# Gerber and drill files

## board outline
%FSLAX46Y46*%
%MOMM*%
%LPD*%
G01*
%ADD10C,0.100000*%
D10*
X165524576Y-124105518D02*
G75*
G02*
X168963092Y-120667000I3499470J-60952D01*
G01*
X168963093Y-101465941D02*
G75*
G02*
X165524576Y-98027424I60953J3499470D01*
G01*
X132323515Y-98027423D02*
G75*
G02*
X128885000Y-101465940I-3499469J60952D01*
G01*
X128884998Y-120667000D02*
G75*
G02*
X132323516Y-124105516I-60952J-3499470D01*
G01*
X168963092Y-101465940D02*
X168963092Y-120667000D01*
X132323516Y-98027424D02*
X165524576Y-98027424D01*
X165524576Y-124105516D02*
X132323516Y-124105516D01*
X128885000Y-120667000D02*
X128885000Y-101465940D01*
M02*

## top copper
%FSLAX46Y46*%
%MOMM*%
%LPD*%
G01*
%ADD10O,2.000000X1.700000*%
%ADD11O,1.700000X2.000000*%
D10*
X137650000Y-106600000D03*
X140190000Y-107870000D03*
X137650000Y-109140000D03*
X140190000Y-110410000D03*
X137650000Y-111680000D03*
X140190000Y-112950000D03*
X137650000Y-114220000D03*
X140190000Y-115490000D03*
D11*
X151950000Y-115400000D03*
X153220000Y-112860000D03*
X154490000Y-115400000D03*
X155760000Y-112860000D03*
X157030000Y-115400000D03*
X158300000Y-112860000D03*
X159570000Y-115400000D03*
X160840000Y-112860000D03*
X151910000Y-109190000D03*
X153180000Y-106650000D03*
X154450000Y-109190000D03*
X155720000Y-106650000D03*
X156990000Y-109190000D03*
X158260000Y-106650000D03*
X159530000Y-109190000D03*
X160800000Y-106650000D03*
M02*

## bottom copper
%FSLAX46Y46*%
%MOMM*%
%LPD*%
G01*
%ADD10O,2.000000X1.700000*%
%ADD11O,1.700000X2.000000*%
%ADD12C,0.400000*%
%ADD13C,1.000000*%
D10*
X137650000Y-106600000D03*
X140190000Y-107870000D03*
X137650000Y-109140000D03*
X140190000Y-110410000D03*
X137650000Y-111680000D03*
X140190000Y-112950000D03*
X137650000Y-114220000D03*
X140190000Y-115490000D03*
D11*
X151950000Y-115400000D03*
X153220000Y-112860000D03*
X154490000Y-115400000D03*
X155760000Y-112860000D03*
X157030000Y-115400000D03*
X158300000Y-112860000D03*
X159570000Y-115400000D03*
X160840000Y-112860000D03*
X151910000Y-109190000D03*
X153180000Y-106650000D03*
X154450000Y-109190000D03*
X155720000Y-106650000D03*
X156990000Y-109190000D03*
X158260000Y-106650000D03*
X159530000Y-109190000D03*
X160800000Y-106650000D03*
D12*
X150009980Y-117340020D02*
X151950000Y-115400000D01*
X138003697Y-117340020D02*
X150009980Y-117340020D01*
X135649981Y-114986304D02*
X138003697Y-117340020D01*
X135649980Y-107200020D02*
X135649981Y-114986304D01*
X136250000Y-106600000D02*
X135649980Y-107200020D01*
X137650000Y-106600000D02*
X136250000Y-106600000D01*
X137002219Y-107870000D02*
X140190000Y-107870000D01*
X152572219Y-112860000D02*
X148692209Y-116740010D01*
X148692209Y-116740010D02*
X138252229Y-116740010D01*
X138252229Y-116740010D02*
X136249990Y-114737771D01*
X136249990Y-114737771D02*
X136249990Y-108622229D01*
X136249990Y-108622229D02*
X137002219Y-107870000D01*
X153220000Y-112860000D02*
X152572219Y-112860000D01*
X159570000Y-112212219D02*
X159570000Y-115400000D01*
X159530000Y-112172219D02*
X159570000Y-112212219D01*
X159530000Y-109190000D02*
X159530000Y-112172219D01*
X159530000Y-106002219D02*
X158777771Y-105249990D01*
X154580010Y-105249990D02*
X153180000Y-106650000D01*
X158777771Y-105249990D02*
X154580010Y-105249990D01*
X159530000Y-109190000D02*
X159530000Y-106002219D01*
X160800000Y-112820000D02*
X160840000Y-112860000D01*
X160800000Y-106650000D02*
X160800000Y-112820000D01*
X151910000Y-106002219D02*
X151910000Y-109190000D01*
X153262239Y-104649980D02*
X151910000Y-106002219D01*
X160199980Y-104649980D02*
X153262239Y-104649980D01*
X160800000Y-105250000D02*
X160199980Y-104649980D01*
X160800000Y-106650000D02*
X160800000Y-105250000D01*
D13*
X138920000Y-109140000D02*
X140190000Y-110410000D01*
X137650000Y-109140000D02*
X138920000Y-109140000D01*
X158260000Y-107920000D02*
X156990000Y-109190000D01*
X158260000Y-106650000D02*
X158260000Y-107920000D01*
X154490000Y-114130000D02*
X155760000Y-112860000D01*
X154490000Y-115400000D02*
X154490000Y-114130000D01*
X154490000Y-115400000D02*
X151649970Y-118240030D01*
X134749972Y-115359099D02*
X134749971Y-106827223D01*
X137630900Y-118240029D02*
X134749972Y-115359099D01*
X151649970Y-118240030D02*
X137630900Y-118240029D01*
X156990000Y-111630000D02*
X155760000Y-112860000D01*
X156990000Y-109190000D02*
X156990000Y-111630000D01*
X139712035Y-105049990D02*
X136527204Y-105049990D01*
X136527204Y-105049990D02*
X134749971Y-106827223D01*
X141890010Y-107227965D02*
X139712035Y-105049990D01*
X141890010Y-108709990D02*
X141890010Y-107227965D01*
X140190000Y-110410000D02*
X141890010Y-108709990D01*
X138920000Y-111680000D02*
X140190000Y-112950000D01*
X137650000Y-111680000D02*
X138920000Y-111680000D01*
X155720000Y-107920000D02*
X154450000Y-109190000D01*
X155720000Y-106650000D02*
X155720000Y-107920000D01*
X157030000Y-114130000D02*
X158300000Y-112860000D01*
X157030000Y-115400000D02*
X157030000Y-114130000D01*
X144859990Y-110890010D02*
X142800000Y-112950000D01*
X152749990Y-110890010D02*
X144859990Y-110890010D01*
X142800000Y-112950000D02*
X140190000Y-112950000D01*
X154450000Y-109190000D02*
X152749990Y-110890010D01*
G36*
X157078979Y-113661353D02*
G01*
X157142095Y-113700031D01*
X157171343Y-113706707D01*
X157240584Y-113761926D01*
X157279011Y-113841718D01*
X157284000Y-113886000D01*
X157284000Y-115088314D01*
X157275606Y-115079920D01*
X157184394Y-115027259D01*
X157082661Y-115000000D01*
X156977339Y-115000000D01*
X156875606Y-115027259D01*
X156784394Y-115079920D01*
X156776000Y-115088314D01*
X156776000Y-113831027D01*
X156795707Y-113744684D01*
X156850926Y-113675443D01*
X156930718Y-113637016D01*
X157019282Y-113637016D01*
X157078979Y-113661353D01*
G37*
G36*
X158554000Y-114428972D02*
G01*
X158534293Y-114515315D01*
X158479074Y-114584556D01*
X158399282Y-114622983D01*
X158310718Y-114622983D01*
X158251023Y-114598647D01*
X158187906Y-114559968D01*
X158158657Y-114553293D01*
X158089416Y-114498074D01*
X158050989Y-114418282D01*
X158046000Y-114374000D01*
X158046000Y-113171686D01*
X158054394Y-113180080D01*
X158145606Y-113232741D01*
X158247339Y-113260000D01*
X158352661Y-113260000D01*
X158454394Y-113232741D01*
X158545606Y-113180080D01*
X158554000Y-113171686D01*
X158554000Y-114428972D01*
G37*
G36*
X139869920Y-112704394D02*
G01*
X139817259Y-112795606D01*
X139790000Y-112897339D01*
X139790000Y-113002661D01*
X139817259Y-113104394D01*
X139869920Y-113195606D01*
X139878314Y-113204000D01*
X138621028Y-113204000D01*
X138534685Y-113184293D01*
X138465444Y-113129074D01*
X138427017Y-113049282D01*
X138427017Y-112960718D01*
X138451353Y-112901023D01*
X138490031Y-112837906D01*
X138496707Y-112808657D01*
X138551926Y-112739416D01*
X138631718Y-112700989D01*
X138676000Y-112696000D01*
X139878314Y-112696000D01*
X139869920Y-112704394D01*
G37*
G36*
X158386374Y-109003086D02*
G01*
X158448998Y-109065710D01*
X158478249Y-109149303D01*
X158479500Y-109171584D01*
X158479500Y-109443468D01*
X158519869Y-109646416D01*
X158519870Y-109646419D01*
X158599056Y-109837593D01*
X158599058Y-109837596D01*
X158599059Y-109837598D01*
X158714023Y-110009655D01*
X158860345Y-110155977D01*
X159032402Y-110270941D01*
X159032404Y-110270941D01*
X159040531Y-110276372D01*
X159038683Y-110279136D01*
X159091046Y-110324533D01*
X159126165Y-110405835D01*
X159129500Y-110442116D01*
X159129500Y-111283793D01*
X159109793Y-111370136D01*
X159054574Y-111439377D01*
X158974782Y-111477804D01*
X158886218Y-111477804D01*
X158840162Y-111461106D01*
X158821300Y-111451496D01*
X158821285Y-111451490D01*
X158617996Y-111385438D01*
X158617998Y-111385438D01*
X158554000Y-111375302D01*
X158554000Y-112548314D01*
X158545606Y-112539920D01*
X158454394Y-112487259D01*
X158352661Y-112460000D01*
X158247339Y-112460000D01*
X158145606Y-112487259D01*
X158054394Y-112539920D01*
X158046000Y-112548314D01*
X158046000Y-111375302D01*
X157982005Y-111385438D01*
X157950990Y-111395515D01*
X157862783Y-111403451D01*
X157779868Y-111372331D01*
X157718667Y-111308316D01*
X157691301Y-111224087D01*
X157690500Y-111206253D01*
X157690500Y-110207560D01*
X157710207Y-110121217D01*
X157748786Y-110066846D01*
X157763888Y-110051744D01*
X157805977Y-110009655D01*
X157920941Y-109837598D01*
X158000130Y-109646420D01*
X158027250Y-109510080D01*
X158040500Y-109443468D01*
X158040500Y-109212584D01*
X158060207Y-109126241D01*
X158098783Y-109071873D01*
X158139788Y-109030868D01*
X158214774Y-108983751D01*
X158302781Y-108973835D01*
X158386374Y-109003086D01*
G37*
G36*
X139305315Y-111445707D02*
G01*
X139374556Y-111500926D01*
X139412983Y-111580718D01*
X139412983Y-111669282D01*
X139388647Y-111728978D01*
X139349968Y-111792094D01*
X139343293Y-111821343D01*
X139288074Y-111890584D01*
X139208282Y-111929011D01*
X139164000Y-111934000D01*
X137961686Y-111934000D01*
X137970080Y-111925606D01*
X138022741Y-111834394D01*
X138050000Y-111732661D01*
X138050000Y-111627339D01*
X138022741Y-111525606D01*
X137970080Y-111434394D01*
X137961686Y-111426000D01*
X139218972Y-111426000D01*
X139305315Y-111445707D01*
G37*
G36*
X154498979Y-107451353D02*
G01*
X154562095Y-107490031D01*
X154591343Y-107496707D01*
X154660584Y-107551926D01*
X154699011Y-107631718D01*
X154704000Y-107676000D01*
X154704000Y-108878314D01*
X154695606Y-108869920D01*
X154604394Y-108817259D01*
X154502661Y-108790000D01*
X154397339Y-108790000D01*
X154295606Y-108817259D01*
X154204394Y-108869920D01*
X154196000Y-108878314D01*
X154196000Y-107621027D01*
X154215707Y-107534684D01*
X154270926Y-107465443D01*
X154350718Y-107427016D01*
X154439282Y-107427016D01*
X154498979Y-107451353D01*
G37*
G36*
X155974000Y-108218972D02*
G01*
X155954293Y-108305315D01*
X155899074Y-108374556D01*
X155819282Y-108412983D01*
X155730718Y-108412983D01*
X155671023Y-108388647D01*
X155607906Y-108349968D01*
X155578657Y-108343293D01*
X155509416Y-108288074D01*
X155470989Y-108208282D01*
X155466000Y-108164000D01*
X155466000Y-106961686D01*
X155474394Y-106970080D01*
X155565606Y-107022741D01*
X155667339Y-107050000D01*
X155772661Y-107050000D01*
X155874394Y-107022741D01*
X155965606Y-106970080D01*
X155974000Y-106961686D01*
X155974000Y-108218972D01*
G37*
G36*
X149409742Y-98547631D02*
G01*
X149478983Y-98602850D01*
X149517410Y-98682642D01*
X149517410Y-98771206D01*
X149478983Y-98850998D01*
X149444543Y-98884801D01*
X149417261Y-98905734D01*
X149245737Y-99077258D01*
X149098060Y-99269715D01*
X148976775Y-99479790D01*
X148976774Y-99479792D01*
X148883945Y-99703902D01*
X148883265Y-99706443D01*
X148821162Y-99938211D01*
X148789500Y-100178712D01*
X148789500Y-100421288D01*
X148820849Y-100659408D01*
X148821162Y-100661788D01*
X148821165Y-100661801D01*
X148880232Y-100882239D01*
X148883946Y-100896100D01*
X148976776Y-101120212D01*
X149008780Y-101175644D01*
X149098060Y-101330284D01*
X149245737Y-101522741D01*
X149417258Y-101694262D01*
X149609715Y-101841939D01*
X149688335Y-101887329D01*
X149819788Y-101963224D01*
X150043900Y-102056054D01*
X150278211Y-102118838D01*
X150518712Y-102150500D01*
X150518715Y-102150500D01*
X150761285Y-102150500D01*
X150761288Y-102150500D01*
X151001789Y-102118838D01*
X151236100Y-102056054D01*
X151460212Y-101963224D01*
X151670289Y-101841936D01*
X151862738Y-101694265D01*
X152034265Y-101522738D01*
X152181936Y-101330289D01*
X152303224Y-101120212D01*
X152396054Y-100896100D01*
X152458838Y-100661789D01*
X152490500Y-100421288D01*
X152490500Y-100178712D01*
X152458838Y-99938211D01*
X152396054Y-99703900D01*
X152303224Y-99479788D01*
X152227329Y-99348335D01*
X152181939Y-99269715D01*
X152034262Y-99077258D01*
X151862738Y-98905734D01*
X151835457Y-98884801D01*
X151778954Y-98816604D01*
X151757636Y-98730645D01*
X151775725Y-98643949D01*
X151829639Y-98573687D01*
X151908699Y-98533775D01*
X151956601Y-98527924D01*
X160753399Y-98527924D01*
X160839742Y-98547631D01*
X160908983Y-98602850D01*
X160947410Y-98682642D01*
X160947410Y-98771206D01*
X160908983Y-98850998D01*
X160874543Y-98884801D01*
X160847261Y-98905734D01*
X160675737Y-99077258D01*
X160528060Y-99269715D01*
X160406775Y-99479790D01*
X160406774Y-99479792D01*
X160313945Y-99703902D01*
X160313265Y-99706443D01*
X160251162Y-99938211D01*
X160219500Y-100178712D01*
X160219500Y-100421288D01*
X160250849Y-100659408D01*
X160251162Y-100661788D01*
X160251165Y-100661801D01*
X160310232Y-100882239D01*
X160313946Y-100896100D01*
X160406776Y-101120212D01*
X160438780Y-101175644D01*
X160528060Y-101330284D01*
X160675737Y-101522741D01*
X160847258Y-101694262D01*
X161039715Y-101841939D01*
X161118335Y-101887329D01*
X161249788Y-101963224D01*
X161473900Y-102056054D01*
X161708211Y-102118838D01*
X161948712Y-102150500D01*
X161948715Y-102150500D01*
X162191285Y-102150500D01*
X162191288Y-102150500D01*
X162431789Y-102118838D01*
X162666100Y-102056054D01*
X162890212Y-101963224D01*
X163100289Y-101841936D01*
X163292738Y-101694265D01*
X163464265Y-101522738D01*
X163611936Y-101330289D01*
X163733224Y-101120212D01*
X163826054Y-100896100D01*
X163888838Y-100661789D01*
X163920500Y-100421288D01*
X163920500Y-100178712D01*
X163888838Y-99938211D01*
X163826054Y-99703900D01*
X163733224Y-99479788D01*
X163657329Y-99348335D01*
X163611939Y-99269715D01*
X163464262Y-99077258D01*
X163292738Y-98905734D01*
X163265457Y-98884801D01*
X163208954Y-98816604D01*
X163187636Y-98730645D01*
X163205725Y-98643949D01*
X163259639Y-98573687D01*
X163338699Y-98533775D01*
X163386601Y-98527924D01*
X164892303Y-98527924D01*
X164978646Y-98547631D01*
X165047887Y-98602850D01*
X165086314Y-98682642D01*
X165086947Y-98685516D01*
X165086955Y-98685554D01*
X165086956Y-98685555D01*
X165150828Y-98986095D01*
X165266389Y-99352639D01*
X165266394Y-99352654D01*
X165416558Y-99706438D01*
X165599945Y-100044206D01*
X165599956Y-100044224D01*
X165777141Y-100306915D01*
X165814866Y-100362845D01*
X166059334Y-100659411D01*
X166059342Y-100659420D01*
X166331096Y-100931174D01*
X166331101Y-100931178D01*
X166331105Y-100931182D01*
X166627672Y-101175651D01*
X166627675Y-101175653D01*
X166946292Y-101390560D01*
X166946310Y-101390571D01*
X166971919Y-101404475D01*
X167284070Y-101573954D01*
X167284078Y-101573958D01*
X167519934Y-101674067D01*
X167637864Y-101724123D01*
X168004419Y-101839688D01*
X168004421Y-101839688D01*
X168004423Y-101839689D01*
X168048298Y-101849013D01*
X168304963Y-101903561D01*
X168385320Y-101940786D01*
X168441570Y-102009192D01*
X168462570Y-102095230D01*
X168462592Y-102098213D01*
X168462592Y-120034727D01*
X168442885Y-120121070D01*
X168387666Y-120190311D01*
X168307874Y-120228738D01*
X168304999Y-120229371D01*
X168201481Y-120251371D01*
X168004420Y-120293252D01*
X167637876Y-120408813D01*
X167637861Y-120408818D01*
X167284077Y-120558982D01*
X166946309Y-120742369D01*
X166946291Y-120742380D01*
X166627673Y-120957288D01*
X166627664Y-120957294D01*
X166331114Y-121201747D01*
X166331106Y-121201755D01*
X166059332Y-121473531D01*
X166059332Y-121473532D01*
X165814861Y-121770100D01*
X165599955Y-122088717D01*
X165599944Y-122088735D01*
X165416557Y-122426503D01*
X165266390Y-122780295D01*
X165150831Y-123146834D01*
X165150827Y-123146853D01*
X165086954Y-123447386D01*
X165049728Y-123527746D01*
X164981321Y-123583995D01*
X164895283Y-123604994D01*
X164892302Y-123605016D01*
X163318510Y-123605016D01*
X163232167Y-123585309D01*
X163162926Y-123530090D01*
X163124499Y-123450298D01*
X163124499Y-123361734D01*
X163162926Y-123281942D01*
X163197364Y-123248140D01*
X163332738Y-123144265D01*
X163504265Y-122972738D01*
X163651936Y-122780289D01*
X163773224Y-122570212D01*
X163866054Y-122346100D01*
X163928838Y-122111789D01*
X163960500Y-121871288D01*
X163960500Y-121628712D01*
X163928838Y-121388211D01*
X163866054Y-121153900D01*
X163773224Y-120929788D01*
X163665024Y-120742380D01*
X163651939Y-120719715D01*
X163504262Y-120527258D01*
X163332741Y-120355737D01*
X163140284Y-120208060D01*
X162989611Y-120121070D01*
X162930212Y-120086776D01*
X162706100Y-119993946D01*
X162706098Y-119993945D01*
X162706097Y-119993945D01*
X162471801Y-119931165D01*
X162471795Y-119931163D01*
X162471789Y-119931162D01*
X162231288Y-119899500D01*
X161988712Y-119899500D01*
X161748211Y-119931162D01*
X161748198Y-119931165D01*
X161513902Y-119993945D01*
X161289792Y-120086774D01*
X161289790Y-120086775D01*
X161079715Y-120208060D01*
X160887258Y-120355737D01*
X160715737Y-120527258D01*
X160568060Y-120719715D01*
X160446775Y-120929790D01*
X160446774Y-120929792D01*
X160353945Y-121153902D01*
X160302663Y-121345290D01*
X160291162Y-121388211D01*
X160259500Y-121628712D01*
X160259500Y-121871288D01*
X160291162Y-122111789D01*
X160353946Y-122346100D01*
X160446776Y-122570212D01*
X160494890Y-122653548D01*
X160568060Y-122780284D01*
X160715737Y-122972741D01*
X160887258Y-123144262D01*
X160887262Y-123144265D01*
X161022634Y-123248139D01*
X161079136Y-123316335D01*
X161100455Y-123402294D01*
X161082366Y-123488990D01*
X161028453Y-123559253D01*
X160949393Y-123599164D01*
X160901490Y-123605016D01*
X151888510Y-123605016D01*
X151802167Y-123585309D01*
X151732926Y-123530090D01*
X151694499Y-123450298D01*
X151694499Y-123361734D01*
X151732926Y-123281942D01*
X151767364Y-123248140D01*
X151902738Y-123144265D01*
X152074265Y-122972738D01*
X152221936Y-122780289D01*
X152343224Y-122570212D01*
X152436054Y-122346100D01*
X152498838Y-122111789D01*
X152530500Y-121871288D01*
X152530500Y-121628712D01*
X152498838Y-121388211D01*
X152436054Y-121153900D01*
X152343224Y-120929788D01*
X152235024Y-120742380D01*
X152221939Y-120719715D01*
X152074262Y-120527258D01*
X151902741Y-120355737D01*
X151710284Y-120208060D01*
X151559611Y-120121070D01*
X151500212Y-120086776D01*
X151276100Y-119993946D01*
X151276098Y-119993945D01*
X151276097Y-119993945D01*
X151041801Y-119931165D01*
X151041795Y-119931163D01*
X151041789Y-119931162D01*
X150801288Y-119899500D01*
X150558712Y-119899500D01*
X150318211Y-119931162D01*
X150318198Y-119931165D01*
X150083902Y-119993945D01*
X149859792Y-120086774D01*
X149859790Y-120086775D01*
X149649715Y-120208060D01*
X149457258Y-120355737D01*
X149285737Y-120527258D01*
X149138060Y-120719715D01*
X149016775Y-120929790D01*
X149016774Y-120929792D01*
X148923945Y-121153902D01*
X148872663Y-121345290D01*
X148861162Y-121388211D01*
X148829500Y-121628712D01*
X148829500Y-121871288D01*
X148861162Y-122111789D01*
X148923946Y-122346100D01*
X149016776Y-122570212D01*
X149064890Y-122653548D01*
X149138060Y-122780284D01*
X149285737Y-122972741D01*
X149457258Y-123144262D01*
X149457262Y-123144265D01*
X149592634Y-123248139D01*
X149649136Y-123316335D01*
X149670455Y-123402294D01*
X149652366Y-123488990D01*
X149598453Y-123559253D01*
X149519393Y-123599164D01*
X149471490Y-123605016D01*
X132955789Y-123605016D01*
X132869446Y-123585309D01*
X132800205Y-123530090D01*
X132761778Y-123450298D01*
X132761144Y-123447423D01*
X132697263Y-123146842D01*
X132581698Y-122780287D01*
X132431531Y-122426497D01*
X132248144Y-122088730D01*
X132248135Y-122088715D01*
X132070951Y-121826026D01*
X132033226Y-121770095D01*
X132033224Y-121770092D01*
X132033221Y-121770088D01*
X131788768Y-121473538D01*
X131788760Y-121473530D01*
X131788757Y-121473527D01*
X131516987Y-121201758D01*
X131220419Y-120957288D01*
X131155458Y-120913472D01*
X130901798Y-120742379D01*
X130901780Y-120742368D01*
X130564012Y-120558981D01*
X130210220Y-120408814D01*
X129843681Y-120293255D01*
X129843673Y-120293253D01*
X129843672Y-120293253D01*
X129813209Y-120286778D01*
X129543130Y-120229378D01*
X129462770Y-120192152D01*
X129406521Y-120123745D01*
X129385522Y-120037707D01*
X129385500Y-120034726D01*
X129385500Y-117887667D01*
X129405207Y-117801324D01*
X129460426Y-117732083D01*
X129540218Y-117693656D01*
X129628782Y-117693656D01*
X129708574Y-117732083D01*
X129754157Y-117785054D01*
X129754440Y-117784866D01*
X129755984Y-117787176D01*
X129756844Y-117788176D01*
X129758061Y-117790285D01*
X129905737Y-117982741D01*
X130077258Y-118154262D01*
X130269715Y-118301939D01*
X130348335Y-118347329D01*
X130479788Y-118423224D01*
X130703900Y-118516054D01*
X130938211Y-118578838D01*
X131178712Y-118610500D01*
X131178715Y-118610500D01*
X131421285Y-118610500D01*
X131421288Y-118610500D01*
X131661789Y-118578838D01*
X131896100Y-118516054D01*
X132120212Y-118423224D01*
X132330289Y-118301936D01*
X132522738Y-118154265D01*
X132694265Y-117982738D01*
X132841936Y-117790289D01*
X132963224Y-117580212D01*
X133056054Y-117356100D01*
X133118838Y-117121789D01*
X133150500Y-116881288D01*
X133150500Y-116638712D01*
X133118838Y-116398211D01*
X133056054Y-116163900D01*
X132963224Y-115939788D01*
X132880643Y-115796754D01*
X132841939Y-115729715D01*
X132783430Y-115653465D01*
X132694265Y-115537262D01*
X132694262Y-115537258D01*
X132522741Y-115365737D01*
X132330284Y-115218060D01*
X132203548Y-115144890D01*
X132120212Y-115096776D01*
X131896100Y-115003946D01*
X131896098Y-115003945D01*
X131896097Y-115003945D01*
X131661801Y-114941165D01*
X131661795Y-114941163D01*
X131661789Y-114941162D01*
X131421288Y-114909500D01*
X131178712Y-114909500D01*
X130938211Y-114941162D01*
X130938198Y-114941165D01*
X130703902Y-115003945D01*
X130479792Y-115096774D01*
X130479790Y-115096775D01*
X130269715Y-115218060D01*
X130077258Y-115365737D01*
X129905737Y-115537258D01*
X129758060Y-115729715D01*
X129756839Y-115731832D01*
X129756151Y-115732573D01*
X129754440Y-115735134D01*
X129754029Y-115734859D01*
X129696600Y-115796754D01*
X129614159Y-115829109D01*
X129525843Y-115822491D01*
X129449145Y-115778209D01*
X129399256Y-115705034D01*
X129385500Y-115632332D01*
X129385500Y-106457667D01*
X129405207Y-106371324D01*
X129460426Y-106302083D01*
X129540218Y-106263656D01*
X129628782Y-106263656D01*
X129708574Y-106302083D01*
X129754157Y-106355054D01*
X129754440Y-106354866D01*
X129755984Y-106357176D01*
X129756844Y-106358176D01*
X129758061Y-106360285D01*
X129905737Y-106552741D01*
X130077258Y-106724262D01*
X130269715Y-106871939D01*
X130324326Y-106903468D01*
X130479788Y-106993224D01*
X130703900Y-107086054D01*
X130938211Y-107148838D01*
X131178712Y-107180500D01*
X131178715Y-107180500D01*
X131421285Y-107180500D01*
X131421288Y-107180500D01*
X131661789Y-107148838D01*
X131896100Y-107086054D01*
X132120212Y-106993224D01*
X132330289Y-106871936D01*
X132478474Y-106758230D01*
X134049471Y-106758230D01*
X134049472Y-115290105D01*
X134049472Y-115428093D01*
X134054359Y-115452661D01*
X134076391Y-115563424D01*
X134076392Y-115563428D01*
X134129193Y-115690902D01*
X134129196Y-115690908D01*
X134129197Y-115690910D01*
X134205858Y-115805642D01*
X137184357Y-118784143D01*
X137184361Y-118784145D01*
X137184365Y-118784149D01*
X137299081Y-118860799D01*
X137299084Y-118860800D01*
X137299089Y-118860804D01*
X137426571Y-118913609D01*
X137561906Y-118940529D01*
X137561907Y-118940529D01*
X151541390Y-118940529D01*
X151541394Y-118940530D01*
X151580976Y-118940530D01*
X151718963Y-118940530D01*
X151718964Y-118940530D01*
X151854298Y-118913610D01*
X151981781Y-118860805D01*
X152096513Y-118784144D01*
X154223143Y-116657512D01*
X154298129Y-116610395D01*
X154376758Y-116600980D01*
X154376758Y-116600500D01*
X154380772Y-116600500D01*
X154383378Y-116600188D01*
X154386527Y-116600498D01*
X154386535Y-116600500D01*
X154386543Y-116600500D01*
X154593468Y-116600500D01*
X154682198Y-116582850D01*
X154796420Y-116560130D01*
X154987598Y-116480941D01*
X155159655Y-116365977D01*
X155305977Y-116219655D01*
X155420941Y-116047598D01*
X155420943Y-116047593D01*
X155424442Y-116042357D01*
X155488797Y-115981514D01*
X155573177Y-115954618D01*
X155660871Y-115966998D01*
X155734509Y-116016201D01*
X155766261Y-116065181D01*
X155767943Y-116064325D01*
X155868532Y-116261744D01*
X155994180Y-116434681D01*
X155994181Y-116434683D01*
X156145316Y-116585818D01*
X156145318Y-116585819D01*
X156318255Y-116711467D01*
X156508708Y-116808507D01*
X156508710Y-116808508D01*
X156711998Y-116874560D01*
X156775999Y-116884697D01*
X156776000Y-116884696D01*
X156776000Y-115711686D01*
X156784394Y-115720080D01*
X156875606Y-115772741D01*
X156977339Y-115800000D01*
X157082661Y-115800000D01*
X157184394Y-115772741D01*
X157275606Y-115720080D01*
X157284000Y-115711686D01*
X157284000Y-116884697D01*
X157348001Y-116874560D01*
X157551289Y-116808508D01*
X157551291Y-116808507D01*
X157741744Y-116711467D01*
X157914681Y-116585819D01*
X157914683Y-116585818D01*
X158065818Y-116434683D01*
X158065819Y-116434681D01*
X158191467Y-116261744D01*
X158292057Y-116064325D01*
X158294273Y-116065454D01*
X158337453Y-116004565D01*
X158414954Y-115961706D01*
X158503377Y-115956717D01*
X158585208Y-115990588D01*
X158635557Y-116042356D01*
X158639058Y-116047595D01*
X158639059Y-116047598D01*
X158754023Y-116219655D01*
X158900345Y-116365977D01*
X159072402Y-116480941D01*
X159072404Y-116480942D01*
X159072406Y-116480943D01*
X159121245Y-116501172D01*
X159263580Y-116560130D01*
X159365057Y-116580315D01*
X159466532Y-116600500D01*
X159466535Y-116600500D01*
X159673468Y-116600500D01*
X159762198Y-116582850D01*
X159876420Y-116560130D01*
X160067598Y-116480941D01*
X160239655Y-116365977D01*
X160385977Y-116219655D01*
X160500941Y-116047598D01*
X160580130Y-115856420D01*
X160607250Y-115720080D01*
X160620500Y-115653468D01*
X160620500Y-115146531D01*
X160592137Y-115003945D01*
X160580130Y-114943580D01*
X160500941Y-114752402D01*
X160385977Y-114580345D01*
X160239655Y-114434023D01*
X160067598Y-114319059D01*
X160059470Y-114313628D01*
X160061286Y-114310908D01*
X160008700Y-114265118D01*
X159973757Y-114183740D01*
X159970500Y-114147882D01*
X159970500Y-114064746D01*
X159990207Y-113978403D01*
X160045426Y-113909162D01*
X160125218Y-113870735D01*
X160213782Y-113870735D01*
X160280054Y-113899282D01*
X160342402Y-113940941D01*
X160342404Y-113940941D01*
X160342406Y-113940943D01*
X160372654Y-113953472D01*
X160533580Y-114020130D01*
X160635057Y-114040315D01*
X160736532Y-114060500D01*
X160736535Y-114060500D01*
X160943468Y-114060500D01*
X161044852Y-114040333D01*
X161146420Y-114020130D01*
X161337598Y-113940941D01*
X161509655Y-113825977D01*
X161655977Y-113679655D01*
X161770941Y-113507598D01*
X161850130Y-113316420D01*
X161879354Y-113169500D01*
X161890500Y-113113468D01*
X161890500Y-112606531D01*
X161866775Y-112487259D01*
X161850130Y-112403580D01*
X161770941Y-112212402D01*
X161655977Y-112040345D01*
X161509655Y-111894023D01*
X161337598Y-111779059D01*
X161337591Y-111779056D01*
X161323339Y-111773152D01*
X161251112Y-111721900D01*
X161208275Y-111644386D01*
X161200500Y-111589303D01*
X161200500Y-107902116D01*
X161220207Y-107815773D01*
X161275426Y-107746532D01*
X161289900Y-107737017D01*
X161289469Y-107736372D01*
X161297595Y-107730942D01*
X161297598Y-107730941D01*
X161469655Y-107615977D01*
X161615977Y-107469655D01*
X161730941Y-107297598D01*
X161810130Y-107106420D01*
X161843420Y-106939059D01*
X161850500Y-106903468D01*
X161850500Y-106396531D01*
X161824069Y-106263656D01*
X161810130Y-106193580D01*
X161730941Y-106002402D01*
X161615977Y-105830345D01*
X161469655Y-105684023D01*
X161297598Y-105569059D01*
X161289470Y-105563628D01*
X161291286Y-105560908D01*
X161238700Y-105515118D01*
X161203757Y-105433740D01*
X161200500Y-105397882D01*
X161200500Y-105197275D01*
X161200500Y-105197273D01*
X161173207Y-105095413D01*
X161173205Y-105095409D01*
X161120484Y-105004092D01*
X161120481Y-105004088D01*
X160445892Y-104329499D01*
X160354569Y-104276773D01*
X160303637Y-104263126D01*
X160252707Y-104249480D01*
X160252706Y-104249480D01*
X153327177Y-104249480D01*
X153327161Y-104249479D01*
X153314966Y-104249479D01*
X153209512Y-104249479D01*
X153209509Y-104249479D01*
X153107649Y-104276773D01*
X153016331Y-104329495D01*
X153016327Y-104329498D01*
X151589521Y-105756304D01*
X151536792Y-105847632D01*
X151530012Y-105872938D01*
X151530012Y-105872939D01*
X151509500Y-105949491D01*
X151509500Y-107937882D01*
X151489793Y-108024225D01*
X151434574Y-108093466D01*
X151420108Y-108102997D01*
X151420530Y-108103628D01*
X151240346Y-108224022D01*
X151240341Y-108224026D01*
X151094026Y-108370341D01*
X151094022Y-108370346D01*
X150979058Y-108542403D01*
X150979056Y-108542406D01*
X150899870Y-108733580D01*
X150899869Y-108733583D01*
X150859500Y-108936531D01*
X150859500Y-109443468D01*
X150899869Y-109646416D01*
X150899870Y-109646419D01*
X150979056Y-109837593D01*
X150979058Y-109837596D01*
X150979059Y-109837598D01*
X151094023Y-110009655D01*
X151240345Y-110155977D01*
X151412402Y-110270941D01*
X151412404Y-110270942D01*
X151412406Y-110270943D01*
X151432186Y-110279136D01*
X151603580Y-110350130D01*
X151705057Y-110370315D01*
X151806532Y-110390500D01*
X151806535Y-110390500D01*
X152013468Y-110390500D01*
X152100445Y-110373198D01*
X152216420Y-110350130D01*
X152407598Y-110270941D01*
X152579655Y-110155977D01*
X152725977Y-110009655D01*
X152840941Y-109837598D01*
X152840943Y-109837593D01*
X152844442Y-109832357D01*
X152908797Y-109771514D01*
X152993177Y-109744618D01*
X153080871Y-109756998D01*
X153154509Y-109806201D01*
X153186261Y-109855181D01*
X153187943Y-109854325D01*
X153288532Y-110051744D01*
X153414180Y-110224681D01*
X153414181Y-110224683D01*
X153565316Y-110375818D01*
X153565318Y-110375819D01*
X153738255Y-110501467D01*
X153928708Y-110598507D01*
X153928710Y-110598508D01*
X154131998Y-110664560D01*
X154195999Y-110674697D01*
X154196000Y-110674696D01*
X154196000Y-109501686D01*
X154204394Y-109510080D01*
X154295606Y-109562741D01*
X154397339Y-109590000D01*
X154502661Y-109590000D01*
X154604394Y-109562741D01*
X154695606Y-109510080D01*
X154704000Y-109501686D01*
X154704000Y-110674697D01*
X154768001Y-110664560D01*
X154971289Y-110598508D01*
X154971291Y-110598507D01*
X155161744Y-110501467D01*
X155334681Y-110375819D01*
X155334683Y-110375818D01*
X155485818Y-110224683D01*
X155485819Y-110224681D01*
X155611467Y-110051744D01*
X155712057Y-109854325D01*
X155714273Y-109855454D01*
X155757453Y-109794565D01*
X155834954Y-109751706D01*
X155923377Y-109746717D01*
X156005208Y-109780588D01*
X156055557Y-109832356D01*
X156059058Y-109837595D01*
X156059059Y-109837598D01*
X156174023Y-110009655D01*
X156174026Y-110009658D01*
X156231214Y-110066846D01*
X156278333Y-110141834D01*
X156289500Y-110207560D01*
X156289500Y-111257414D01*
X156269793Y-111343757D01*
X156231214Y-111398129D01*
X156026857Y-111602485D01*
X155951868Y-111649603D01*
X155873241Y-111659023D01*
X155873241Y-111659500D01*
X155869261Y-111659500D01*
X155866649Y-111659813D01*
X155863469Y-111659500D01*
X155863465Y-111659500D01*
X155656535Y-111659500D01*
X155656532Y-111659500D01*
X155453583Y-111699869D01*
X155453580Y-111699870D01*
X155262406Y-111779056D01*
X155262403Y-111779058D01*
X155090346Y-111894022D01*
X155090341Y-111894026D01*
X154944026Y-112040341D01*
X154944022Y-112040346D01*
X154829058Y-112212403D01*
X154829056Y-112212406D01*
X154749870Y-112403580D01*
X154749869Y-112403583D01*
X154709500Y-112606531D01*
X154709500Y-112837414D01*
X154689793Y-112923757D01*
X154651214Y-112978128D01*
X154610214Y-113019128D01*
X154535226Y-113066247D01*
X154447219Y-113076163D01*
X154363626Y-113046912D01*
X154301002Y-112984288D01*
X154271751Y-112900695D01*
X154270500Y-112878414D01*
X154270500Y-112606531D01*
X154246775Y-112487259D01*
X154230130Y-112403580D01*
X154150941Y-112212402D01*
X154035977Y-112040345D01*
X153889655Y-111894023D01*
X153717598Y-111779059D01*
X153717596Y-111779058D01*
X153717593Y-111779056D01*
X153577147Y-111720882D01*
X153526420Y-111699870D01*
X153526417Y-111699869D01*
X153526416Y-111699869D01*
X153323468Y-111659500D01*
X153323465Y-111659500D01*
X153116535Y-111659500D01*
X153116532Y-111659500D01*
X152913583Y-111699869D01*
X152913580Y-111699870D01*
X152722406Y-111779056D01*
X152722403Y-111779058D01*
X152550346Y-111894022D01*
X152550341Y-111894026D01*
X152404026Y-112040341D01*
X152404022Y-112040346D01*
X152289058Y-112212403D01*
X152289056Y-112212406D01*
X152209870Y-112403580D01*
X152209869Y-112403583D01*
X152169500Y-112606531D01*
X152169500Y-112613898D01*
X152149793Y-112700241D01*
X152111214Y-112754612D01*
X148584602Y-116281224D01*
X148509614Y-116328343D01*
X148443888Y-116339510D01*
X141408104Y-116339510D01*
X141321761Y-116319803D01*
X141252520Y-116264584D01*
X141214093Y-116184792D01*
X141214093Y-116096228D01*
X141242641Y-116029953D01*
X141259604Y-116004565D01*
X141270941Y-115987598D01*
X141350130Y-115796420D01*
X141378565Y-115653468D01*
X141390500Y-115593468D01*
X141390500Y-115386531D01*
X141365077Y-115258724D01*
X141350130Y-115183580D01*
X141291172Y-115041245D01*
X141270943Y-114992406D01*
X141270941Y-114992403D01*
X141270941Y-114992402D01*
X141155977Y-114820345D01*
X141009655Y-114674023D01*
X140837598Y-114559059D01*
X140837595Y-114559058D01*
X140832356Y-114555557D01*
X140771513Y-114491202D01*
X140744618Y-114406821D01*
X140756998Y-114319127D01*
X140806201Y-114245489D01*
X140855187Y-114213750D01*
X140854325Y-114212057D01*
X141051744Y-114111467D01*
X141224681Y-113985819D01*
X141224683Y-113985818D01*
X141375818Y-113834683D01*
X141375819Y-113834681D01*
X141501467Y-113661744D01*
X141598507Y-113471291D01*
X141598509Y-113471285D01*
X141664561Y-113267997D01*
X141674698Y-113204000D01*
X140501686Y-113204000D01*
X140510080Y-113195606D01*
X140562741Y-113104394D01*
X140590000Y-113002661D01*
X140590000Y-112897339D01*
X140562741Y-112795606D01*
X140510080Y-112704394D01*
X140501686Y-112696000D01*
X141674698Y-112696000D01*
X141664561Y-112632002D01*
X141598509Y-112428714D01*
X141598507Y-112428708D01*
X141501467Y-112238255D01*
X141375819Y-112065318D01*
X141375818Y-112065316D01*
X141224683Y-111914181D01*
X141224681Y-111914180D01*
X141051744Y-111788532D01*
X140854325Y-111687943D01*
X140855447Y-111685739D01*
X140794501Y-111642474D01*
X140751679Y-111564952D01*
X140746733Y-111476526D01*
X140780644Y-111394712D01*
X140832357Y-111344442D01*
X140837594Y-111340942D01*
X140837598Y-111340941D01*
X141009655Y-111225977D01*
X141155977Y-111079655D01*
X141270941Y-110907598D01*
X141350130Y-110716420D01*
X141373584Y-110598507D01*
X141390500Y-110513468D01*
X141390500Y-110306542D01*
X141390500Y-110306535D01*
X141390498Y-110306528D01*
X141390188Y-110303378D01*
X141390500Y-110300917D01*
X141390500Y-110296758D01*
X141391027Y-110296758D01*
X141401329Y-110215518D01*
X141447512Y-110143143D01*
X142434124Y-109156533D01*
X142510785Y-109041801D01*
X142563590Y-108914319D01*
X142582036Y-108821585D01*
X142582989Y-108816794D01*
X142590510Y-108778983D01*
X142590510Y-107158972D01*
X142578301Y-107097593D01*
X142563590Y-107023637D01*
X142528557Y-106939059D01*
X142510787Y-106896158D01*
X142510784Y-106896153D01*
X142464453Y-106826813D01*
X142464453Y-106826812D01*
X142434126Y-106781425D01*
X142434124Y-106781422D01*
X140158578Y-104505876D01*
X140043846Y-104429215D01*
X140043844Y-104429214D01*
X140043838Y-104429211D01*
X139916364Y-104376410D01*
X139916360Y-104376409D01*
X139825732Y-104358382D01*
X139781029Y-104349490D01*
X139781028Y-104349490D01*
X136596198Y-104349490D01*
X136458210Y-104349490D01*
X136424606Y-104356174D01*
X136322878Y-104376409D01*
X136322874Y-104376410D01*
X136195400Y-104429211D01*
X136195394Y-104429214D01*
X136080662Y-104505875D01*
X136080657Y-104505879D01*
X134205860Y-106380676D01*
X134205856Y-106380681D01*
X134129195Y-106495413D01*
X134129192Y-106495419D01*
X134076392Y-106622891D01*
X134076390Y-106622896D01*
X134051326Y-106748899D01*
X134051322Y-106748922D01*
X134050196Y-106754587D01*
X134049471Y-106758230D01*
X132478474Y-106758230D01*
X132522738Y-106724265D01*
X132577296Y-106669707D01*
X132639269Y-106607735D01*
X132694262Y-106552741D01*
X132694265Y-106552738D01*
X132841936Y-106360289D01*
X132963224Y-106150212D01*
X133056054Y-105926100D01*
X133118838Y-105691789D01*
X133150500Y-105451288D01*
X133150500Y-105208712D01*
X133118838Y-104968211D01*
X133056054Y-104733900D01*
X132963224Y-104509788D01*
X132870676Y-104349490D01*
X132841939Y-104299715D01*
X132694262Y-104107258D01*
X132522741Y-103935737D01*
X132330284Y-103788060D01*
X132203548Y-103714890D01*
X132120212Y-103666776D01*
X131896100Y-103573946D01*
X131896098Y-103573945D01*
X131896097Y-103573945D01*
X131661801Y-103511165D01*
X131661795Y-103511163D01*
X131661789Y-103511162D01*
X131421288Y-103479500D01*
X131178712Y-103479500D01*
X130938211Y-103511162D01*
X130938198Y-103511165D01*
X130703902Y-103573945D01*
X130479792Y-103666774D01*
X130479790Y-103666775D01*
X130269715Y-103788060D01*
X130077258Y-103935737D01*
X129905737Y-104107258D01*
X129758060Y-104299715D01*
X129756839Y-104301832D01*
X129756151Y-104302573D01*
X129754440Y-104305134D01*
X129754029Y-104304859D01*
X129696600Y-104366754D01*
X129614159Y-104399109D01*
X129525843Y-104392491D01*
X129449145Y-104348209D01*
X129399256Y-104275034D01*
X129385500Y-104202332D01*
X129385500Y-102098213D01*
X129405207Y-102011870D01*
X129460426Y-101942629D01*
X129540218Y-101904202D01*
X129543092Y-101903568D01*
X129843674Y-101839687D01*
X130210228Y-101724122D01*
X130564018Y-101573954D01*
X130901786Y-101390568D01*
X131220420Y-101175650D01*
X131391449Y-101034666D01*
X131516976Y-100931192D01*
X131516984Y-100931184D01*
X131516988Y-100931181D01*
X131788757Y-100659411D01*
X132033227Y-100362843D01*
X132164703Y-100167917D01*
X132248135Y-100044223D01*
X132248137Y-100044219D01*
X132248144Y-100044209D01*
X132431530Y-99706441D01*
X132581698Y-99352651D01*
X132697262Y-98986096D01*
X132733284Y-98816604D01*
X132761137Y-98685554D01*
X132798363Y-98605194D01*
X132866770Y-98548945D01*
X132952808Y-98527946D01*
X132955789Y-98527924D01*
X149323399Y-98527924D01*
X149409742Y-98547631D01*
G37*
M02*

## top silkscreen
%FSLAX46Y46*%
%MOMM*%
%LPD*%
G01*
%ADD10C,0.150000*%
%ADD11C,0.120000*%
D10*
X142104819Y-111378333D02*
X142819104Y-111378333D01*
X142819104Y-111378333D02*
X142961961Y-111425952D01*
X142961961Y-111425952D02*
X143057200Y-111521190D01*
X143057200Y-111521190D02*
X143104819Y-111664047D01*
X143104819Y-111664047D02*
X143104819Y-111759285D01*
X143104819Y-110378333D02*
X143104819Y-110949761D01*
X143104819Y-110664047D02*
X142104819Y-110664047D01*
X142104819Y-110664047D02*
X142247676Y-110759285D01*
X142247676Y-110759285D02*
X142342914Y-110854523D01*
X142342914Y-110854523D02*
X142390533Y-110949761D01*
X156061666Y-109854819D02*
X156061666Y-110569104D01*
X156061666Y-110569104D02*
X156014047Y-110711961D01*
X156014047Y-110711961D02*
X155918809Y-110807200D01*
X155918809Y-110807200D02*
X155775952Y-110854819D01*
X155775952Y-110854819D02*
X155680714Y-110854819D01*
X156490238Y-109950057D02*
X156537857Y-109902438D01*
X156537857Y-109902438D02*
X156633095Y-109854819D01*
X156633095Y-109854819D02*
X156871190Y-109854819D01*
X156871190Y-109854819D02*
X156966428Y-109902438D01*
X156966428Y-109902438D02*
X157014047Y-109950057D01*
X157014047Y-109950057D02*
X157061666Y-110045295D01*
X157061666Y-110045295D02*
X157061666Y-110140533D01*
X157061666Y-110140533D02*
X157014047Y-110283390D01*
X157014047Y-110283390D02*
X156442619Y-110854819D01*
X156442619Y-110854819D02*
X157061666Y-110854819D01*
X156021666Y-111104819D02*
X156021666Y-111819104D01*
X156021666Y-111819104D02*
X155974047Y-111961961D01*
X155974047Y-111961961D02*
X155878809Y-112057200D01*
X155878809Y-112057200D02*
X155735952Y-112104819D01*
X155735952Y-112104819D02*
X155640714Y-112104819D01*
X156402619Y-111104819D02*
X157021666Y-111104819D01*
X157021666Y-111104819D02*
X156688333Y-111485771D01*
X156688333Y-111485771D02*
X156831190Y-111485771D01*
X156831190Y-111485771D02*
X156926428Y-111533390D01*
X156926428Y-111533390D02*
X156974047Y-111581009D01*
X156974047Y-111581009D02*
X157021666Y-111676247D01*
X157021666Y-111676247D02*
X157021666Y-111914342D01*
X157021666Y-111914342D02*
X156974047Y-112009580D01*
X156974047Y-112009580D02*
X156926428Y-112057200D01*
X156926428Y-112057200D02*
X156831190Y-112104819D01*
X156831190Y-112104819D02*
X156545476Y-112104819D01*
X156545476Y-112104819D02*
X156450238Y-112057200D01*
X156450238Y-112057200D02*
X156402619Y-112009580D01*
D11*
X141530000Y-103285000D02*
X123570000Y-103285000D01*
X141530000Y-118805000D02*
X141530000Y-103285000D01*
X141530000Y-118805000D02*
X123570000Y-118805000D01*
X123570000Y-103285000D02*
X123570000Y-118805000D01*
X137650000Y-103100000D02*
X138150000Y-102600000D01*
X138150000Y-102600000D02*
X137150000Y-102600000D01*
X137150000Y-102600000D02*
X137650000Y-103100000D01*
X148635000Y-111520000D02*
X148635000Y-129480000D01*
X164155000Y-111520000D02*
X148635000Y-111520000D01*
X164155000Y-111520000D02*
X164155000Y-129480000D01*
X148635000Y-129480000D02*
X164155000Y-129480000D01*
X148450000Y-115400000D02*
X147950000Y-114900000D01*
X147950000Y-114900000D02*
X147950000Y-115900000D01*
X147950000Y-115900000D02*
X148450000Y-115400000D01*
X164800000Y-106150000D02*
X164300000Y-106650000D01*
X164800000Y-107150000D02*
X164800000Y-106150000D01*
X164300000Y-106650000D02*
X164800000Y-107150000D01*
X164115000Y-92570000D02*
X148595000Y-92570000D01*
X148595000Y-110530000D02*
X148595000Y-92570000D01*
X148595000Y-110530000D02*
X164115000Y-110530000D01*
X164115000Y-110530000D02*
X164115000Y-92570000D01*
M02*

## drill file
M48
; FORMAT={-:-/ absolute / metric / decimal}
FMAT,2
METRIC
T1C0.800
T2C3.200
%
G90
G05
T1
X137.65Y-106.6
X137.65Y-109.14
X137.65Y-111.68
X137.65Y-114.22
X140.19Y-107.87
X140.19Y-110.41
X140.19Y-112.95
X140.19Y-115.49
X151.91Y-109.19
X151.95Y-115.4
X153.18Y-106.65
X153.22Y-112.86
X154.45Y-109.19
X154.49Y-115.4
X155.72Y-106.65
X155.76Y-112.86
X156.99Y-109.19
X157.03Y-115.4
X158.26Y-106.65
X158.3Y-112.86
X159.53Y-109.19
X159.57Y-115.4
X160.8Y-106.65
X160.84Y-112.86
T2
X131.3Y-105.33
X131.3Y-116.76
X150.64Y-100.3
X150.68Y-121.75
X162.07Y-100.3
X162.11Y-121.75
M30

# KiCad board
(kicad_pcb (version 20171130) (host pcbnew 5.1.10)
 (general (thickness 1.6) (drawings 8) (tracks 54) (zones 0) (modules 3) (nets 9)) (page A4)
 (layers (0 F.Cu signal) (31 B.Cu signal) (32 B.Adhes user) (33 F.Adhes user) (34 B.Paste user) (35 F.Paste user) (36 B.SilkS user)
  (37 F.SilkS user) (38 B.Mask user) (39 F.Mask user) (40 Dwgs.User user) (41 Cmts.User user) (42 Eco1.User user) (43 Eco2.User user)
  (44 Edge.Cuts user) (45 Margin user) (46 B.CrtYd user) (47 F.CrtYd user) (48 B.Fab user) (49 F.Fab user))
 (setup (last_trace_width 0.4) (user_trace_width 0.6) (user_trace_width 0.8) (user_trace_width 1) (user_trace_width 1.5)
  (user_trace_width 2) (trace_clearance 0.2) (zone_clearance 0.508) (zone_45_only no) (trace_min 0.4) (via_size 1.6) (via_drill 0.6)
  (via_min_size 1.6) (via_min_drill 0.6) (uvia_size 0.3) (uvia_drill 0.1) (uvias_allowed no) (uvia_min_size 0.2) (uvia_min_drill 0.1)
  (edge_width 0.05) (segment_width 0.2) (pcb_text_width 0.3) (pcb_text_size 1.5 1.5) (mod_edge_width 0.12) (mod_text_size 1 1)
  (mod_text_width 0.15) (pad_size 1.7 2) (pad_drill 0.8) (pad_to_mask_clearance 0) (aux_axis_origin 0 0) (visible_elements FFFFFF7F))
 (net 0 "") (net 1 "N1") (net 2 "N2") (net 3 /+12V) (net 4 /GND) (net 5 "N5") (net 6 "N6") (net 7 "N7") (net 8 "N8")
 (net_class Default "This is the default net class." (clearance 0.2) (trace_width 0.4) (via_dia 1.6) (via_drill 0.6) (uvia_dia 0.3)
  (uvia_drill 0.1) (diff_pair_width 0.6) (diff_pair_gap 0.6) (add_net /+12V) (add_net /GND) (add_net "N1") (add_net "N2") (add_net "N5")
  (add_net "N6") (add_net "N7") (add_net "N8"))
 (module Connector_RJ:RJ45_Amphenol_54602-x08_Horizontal (layer F.Cu) (at 137.65 106.6 270)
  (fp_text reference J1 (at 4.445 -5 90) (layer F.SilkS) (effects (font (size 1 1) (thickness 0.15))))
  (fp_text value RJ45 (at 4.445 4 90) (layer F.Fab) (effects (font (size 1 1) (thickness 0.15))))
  (fp_line (start -3.315 -3.88) (end -3.315 14.08) (layer F.SilkS) (width 0.12))
  (fp_line (start 12.205 -3.88) (end -3.315 -3.88) (layer F.SilkS) (width 0.12))
  (fp_line (start 12.205 -3.88) (end 12.205 14.08) (layer F.SilkS) (width 0.12))
  (fp_line (start -3.315 14.08) (end 12.205 14.08) (layer F.SilkS) (width 0.12))
  (fp_line (start -3.5 0) (end -4 -0.5) (layer F.SilkS) (width 0.12))
  (fp_line (start -4 -0.5) (end -4 0.5) (layer F.SilkS) (width 0.12))
  (fp_line (start -4 0.5) (end -3.5 0) (layer F.SilkS) (width 0.12))
  (pad "" np_thru_hole circle (at 10.16 6.35 270) (size 3.2 3.2) (drill 3.2) (layers *.Cu *.Mask))
  (pad "" np_thru_hole circle (at -1.27 6.35 270) (size 3.2 3.2) (drill 3.2) (layers *.Cu *.Mask))
  (pad 1 thru_hole oval (at 0 0 270) (size 1.7 2) (drill 0.8) (layers *.Cu *.Mask) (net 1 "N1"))
  (pad 2 thru_hole oval (at 1.27 -2.54 270) (size 1.7 2) (drill 0.8) (layers *.Cu *.Mask) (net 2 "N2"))
  (pad 3 thru_hole oval (at 2.54 0 270) (size 1.7 2) (drill 0.8) (layers *.Cu *.Mask) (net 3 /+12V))
  (pad 4 thru_hole oval (at 3.81 -2.54 270) (size 1.7 2) (drill 0.8) (layers *.Cu *.Mask) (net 3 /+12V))
  (pad 5 thru_hole oval (at 5.08 0 270) (size 1.7 2) (drill 0.8) (layers *.Cu *.Mask) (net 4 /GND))
  (pad 6 thru_hole oval (at 6.35 -2.54 270) (size 1.7 2) (drill 0.8) (layers *.Cu *.Mask) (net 4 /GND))
  (pad 7 thru_hole oval (at 7.62 0 270) (size 1.7 2) (drill 0.8) (layers *.Cu *.Mask) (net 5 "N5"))
  (pad 8 thru_hole oval (at 8.89 -2.54 270) (size 1.7 2) (drill 0.8) (layers *.Cu *.Mask) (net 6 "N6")))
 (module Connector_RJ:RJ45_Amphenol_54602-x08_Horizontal (layer F.Cu) (at 151.95 115.4)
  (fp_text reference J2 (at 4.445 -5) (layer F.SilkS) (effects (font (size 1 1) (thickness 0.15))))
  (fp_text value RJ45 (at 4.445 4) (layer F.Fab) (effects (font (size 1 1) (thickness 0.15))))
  (fp_line (start -3.315 -3.88) (end -3.315 14.08) (layer F.SilkS) (width 0.12))
  (fp_line (start 12.205 -3.88) (end -3.315 -3.88) (layer F.SilkS) (width 0.12))
  (fp_line (start 12.205 -3.88) (end 12.205 14.08) (layer F.SilkS) (width 0.12))
  (fp_line (start -3.315 14.08) (end 12.205 14.08) (layer F.SilkS) (width 0.12))
  (fp_line (start -3.5 0) (end -4 -0.5) (layer F.SilkS) (width 0.12))
  (fp_line (start -4 -0.5) (end -4 0.5) (layer F.SilkS) (width 0.12))
  (fp_line (start -4 0.5) (end -3.5 0) (layer F.SilkS) (width 0.12))
  (pad "" np_thru_hole circle (at 10.16 6.35) (size 3.2 3.2) (drill 3.2) (layers *.Cu *.Mask))
  (pad "" np_thru_hole circle (at -1.27 6.35) (size 3.2 3.2) (drill 3.2) (layers *.Cu *.Mask))
  (pad 1 thru_hole oval (at 0 0) (size 1.7 2) (drill 0.8) (layers *.Cu *.Mask) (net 1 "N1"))
  (pad 2 thru_hole oval (at 1.27 -2.54) (size 1.7 2) (drill 0.8) (layers *.Cu *.Mask) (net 2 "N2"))
  (pad 3 thru_hole oval (at 2.54 0) (size 1.7 2) (drill 0.8) (layers *.Cu *.Mask) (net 3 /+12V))
  (pad 4 thru_hole oval (at 3.81 -2.54) (size 1.7 2) (drill 0.8) (layers *.Cu *.Mask) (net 3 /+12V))
  (pad 5 thru_hole oval (at 5.08 0) (size 1.7 2) (drill 0.8) (layers *.Cu *.Mask) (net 4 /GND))
  (pad 6 thru_hole oval (at 6.35 -2.54) (size 1.7 2) (drill 0.8) (layers *.Cu *.Mask) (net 4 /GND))
  (pad 7 thru_hole oval (at 7.62 0) (size 1.7 2) (drill 0.8) (layers *.Cu *.Mask) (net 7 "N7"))
  (pad 8 thru_hole oval (at 8.89 -2.54) (size 1.7 2) (drill 0.8) (layers *.Cu *.Mask) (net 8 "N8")))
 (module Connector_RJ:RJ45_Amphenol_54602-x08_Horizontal (layer F.Cu) (at 160.8 106.65 180)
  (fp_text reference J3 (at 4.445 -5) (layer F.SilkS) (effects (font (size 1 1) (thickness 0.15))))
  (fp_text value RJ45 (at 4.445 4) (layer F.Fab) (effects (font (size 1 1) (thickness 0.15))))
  (fp_line (start -4 0.5) (end -3.5 0) (layer F.SilkS) (width 0.12))
  (fp_line (start -4 -0.5) (end -4 0.5) (layer F.SilkS) (width 0.12))
  (fp_line (start -3.5 0) (end -4 -0.5) (layer F.SilkS) (width 0.12))
  (fp_line (start -3.315 14.08) (end 12.205 14.08) (layer F.SilkS) (width 0.12))
  (fp_line (start 12.205 -3.88) (end 12.205 14.08) (layer F.SilkS) (width 0.12))
  (fp_line (start 12.205 -3.88) (end -3.315 -3.88) (layer F.SilkS) (width 0.12))
  (fp_line (start -3.315 -3.88) (end -3.315 14.08) (layer F.SilkS) (width 0.12))
  (pad 8 thru_hole oval (at 8.89 -2.54 180) (size 1.7 2) (drill 0.8) (layers *.Cu *.Mask) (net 8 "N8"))
  (pad 7 thru_hole oval (at 7.62 0 180) (size 1.7 2) (drill 0.8) (layers *.Cu *.Mask) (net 7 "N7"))
  (pad 6 thru_hole oval (at 6.35 -2.54 180) (size 1.7 2) (drill 0.8) (layers *.Cu *.Mask) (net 4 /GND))
  (pad 5 thru_hole oval (at 5.08 0 180) (size 1.7 2) (drill 0.8) (layers *.Cu *.Mask) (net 4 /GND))
  (pad 4 thru_hole oval (at 3.81 -2.54 180) (size 1.7 2) (drill 0.8) (layers *.Cu *.Mask) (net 3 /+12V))
  (pad 3 thru_hole oval (at 2.54 0 180) (size 1.7 2) (drill 0.8) (layers *.Cu *.Mask) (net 3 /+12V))
  (pad 2 thru_hole oval (at 1.27 -2.54 180) (size 1.7 2) (drill 0.8) (layers *.Cu *.Mask) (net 7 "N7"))
  (pad 1 thru_hole oval (at 0 0 180) (size 1.7 2) (drill 0.8) (layers *.Cu *.Mask) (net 8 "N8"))
  (pad "" np_thru_hole circle (at -1.27 6.35 180) (size 3.2 3.2) (drill 3.2) (layers *.Cu *.Mask))
  (pad "" np_thru_hole circle (at 10.16 6.35 180) (size 3.2 3.2) (drill 3.2) (layers *.Cu *.Mask)))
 (gr_arc (start 169.024046 124.16647) (end 168.963092 120.667) (angle -88.00426351) (layer Edge.Cuts) (width 0.1))
 (gr_arc (start 169.024046 97.966471) (end 165.524576 98.027424) (angle -88.00426351) (layer Edge.Cuts) (width 0.1))
 (gr_arc (start 128.824046 97.966471) (end 128.885 101.46594) (angle -88.00426351) (layer Edge.Cuts) (width 0.1))
 (gr_arc (start 128.824046 124.16647) (end 132.323516 124.105516) (angle -88.00426351) (layer Edge.Cuts) (width 0.1))
 (gr_line (start 168.963092 101.46594) (end 168.963092 120.667) (layer Edge.Cuts) (width 0.1))
 (gr_line (start 132.323516 98.027424) (end 165.524576 98.027424) (layer Edge.Cuts) (width 0.1))
 (gr_line (start 165.524576 124.105516) (end 132.323516 124.105516) (layer Edge.Cuts) (width 0.1))
 (gr_line (start 128.885 120.667) (end 128.885 101.46594) (layer Edge.Cuts) (width 0.1))
 (segment (start 150.00998 117.34002) (end 151.95 115.4) (width 0.4) (layer B.Cu) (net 1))
 (segment (start 138.003697 117.34002) (end 150.00998 117.34002) (width 0.4) (layer B.Cu) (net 1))
 (segment (start 135.649981 114.986304) (end 138.003697 117.34002) (width 0.4) (layer B.Cu) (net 1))
 (segment (start 135.64998 107.20002) (end 135.649981 114.986304) (width 0.4) (layer B.Cu) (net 1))
 (segment (start 136.25 106.6) (end 135.64998 107.20002) (width 0.4) (layer B.Cu) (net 1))
 (segment (start 137.65 106.6) (end 136.25 106.6) (width 0.4) (layer B.Cu) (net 1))
 (segment (start 137.002219 107.87) (end 140.19 107.87) (width 0.4) (layer B.Cu) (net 2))
 (segment (start 152.572219 112.86) (end 148.692209 116.74001) (width 0.4) (layer B.Cu) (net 2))
 (segment (start 148.692209 116.74001) (end 138.252229 116.74001) (width 0.4) (layer B.Cu) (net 2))
 (segment (start 138.252229 116.74001) (end 136.24999 114.737771) (width 0.4) (layer B.Cu) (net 2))
 (segment (start 136.24999 114.737771) (end 136.24999 108.622229) (width 0.4) (layer B.Cu) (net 2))
 (segment (start 136.24999 108.622229) (end 137.002219 107.87) (width 0.4) (layer B.Cu) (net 2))
 (segment (start 153.22 112.86) (end 152.572219 112.86) (width 0.4) (layer B.Cu) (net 2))
 (segment (start 159.57 112.212219) (end 159.57 115.4) (width 0.4) (layer B.Cu) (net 7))
 (segment (start 159.53 112.172219) (end 159.57 112.212219) (width 0.4) (layer B.Cu) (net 7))
 (segment (start 159.53 109.19) (end 159.53 112.172219) (width 0.4) (layer B.Cu) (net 7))
 (segment (start 159.53 106.002219) (end 158.777771 105.24999) (width 0.4) (layer B.Cu) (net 7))
 (segment (start 154.58001 105.24999) (end 153.18 106.65) (width 0.4) (layer B.Cu) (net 7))
 (segment (start 158.777771 105.24999) (end 154.58001 105.24999) (width 0.4) (layer B.Cu) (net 7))
 (segment (start 159.53 109.19) (end 159.53 106.002219) (width 0.4) (layer B.Cu) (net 7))
 (segment (start 160.8 112.82) (end 160.84 112.86) (width 0.4) (layer B.Cu) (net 8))
 (segment (start 160.8 106.65) (end 160.8 112.82) (width 0.4) (layer B.Cu) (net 8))
 (segment (start 151.91 106.002219) (end 151.91 109.19) (width 0.4) (layer B.Cu) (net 8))
 (segment (start 153.262239 104.64998) (end 151.91 106.002219) (width 0.4) (layer B.Cu) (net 8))
 (segment (start 160.19998 104.64998) (end 153.262239 104.64998) (width 0.4) (layer B.Cu) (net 8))
 (segment (start 160.8 105.25) (end 160.19998 104.64998) (width 0.4) (layer B.Cu) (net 8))
 (segment (start 160.8 106.65) (end 160.8 105.25) (width 0.4) (layer B.Cu) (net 8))
 (segment (start 138.92 109.14) (end 140.19 110.41) (width 1) (layer B.Cu) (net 3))
 (segment (start 137.65 109.14) (end 138.92 109.14) (width 1) (layer B.Cu) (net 3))
 (segment (start 158.26 107.92) (end 156.99 109.19) (width 1) (layer B.Cu) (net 3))
 (segment (start 158.26 106.65) (end 158.26 107.92) (width 1) (layer B.Cu) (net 3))
 (segment (start 154.49 114.13) (end 155.76 112.86) (width 1) (layer B.Cu) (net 3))
 (segment (start 154.49 115.4) (end 154.49 114.13) (width 1) (layer B.Cu) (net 3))
 (segment (start 154.49 115.4) (end 151.64997 118.24003) (width 1) (layer B.Cu) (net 3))
 (segment (start 134.749972 115.359099) (end 134.749971 106.827223) (width 1) (layer B.Cu) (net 3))
 (segment (start 137.6309 118.240029) (end 134.749972 115.359099) (width 1) (layer B.Cu) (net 3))
 (segment (start 151.64997 118.24003) (end 137.6309 118.240029) (width 1) (layer B.Cu) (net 3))
 (segment (start 156.99 111.63) (end 155.76 112.86) (width 1) (layer B.Cu) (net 3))
 (segment (start 156.99 109.19) (end 156.99 111.63) (width 1) (layer B.Cu) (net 3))
 (segment (start 139.712035 105.04999) (end 136.527204 105.04999) (width 1) (layer B.Cu) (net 3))
 (segment (start 136.527204 105.04999) (end 134.749971 106.827223) (width 1) (layer B.Cu) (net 3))
 (segment (start 141.89001 107.227965) (end 139.712035 105.04999) (width 1) (layer B.Cu) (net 3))
 (segment (start 141.89001 108.70999) (end 141.89001 107.227965) (width 1) (layer B.Cu) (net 3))
 (segment (start 140.19 110.41) (end 141.89001 108.70999) (width 1) (layer B.Cu) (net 3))
 (segment (start 138.92 111.68) (end 140.19 112.95) (width 1) (layer B.Cu) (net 4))
 (segment (start 137.65 111.68) (end 138.92 111.68) (width 1) (layer B.Cu) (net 4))
 (segment (start 155.72 107.92) (end 154.45 109.19) (width 1) (layer B.Cu) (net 4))
 (segment (start 155.72 106.65) (end 155.72 107.92) (width 1) (layer B.Cu) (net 4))
 (segment (start 157.03 114.13) (end 158.3 112.86) (width 1) (layer B.Cu) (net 4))
 (segment (start 157.03 115.4) (end 157.03 114.13) (width 1) (layer B.Cu) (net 4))
 (segment (start 144.85999 110.89001) (end 142.8 112.95) (width 1) (layer B.Cu) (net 4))
 (segment (start 152.74999 110.89001) (end 144.85999 110.89001) (width 1) (layer B.Cu) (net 4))
 (segment (start 142.8 112.95) (end 140.19 112.95) (width 1) (layer B.Cu) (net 4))
 (segment (start 154.45 109.19) (end 152.74999 110.89001) (width 1) (layer B.Cu) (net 4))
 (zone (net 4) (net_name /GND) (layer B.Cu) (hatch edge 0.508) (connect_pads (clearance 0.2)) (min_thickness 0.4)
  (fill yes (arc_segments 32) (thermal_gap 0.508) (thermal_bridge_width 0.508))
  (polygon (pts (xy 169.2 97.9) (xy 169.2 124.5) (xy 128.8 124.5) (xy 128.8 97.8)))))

